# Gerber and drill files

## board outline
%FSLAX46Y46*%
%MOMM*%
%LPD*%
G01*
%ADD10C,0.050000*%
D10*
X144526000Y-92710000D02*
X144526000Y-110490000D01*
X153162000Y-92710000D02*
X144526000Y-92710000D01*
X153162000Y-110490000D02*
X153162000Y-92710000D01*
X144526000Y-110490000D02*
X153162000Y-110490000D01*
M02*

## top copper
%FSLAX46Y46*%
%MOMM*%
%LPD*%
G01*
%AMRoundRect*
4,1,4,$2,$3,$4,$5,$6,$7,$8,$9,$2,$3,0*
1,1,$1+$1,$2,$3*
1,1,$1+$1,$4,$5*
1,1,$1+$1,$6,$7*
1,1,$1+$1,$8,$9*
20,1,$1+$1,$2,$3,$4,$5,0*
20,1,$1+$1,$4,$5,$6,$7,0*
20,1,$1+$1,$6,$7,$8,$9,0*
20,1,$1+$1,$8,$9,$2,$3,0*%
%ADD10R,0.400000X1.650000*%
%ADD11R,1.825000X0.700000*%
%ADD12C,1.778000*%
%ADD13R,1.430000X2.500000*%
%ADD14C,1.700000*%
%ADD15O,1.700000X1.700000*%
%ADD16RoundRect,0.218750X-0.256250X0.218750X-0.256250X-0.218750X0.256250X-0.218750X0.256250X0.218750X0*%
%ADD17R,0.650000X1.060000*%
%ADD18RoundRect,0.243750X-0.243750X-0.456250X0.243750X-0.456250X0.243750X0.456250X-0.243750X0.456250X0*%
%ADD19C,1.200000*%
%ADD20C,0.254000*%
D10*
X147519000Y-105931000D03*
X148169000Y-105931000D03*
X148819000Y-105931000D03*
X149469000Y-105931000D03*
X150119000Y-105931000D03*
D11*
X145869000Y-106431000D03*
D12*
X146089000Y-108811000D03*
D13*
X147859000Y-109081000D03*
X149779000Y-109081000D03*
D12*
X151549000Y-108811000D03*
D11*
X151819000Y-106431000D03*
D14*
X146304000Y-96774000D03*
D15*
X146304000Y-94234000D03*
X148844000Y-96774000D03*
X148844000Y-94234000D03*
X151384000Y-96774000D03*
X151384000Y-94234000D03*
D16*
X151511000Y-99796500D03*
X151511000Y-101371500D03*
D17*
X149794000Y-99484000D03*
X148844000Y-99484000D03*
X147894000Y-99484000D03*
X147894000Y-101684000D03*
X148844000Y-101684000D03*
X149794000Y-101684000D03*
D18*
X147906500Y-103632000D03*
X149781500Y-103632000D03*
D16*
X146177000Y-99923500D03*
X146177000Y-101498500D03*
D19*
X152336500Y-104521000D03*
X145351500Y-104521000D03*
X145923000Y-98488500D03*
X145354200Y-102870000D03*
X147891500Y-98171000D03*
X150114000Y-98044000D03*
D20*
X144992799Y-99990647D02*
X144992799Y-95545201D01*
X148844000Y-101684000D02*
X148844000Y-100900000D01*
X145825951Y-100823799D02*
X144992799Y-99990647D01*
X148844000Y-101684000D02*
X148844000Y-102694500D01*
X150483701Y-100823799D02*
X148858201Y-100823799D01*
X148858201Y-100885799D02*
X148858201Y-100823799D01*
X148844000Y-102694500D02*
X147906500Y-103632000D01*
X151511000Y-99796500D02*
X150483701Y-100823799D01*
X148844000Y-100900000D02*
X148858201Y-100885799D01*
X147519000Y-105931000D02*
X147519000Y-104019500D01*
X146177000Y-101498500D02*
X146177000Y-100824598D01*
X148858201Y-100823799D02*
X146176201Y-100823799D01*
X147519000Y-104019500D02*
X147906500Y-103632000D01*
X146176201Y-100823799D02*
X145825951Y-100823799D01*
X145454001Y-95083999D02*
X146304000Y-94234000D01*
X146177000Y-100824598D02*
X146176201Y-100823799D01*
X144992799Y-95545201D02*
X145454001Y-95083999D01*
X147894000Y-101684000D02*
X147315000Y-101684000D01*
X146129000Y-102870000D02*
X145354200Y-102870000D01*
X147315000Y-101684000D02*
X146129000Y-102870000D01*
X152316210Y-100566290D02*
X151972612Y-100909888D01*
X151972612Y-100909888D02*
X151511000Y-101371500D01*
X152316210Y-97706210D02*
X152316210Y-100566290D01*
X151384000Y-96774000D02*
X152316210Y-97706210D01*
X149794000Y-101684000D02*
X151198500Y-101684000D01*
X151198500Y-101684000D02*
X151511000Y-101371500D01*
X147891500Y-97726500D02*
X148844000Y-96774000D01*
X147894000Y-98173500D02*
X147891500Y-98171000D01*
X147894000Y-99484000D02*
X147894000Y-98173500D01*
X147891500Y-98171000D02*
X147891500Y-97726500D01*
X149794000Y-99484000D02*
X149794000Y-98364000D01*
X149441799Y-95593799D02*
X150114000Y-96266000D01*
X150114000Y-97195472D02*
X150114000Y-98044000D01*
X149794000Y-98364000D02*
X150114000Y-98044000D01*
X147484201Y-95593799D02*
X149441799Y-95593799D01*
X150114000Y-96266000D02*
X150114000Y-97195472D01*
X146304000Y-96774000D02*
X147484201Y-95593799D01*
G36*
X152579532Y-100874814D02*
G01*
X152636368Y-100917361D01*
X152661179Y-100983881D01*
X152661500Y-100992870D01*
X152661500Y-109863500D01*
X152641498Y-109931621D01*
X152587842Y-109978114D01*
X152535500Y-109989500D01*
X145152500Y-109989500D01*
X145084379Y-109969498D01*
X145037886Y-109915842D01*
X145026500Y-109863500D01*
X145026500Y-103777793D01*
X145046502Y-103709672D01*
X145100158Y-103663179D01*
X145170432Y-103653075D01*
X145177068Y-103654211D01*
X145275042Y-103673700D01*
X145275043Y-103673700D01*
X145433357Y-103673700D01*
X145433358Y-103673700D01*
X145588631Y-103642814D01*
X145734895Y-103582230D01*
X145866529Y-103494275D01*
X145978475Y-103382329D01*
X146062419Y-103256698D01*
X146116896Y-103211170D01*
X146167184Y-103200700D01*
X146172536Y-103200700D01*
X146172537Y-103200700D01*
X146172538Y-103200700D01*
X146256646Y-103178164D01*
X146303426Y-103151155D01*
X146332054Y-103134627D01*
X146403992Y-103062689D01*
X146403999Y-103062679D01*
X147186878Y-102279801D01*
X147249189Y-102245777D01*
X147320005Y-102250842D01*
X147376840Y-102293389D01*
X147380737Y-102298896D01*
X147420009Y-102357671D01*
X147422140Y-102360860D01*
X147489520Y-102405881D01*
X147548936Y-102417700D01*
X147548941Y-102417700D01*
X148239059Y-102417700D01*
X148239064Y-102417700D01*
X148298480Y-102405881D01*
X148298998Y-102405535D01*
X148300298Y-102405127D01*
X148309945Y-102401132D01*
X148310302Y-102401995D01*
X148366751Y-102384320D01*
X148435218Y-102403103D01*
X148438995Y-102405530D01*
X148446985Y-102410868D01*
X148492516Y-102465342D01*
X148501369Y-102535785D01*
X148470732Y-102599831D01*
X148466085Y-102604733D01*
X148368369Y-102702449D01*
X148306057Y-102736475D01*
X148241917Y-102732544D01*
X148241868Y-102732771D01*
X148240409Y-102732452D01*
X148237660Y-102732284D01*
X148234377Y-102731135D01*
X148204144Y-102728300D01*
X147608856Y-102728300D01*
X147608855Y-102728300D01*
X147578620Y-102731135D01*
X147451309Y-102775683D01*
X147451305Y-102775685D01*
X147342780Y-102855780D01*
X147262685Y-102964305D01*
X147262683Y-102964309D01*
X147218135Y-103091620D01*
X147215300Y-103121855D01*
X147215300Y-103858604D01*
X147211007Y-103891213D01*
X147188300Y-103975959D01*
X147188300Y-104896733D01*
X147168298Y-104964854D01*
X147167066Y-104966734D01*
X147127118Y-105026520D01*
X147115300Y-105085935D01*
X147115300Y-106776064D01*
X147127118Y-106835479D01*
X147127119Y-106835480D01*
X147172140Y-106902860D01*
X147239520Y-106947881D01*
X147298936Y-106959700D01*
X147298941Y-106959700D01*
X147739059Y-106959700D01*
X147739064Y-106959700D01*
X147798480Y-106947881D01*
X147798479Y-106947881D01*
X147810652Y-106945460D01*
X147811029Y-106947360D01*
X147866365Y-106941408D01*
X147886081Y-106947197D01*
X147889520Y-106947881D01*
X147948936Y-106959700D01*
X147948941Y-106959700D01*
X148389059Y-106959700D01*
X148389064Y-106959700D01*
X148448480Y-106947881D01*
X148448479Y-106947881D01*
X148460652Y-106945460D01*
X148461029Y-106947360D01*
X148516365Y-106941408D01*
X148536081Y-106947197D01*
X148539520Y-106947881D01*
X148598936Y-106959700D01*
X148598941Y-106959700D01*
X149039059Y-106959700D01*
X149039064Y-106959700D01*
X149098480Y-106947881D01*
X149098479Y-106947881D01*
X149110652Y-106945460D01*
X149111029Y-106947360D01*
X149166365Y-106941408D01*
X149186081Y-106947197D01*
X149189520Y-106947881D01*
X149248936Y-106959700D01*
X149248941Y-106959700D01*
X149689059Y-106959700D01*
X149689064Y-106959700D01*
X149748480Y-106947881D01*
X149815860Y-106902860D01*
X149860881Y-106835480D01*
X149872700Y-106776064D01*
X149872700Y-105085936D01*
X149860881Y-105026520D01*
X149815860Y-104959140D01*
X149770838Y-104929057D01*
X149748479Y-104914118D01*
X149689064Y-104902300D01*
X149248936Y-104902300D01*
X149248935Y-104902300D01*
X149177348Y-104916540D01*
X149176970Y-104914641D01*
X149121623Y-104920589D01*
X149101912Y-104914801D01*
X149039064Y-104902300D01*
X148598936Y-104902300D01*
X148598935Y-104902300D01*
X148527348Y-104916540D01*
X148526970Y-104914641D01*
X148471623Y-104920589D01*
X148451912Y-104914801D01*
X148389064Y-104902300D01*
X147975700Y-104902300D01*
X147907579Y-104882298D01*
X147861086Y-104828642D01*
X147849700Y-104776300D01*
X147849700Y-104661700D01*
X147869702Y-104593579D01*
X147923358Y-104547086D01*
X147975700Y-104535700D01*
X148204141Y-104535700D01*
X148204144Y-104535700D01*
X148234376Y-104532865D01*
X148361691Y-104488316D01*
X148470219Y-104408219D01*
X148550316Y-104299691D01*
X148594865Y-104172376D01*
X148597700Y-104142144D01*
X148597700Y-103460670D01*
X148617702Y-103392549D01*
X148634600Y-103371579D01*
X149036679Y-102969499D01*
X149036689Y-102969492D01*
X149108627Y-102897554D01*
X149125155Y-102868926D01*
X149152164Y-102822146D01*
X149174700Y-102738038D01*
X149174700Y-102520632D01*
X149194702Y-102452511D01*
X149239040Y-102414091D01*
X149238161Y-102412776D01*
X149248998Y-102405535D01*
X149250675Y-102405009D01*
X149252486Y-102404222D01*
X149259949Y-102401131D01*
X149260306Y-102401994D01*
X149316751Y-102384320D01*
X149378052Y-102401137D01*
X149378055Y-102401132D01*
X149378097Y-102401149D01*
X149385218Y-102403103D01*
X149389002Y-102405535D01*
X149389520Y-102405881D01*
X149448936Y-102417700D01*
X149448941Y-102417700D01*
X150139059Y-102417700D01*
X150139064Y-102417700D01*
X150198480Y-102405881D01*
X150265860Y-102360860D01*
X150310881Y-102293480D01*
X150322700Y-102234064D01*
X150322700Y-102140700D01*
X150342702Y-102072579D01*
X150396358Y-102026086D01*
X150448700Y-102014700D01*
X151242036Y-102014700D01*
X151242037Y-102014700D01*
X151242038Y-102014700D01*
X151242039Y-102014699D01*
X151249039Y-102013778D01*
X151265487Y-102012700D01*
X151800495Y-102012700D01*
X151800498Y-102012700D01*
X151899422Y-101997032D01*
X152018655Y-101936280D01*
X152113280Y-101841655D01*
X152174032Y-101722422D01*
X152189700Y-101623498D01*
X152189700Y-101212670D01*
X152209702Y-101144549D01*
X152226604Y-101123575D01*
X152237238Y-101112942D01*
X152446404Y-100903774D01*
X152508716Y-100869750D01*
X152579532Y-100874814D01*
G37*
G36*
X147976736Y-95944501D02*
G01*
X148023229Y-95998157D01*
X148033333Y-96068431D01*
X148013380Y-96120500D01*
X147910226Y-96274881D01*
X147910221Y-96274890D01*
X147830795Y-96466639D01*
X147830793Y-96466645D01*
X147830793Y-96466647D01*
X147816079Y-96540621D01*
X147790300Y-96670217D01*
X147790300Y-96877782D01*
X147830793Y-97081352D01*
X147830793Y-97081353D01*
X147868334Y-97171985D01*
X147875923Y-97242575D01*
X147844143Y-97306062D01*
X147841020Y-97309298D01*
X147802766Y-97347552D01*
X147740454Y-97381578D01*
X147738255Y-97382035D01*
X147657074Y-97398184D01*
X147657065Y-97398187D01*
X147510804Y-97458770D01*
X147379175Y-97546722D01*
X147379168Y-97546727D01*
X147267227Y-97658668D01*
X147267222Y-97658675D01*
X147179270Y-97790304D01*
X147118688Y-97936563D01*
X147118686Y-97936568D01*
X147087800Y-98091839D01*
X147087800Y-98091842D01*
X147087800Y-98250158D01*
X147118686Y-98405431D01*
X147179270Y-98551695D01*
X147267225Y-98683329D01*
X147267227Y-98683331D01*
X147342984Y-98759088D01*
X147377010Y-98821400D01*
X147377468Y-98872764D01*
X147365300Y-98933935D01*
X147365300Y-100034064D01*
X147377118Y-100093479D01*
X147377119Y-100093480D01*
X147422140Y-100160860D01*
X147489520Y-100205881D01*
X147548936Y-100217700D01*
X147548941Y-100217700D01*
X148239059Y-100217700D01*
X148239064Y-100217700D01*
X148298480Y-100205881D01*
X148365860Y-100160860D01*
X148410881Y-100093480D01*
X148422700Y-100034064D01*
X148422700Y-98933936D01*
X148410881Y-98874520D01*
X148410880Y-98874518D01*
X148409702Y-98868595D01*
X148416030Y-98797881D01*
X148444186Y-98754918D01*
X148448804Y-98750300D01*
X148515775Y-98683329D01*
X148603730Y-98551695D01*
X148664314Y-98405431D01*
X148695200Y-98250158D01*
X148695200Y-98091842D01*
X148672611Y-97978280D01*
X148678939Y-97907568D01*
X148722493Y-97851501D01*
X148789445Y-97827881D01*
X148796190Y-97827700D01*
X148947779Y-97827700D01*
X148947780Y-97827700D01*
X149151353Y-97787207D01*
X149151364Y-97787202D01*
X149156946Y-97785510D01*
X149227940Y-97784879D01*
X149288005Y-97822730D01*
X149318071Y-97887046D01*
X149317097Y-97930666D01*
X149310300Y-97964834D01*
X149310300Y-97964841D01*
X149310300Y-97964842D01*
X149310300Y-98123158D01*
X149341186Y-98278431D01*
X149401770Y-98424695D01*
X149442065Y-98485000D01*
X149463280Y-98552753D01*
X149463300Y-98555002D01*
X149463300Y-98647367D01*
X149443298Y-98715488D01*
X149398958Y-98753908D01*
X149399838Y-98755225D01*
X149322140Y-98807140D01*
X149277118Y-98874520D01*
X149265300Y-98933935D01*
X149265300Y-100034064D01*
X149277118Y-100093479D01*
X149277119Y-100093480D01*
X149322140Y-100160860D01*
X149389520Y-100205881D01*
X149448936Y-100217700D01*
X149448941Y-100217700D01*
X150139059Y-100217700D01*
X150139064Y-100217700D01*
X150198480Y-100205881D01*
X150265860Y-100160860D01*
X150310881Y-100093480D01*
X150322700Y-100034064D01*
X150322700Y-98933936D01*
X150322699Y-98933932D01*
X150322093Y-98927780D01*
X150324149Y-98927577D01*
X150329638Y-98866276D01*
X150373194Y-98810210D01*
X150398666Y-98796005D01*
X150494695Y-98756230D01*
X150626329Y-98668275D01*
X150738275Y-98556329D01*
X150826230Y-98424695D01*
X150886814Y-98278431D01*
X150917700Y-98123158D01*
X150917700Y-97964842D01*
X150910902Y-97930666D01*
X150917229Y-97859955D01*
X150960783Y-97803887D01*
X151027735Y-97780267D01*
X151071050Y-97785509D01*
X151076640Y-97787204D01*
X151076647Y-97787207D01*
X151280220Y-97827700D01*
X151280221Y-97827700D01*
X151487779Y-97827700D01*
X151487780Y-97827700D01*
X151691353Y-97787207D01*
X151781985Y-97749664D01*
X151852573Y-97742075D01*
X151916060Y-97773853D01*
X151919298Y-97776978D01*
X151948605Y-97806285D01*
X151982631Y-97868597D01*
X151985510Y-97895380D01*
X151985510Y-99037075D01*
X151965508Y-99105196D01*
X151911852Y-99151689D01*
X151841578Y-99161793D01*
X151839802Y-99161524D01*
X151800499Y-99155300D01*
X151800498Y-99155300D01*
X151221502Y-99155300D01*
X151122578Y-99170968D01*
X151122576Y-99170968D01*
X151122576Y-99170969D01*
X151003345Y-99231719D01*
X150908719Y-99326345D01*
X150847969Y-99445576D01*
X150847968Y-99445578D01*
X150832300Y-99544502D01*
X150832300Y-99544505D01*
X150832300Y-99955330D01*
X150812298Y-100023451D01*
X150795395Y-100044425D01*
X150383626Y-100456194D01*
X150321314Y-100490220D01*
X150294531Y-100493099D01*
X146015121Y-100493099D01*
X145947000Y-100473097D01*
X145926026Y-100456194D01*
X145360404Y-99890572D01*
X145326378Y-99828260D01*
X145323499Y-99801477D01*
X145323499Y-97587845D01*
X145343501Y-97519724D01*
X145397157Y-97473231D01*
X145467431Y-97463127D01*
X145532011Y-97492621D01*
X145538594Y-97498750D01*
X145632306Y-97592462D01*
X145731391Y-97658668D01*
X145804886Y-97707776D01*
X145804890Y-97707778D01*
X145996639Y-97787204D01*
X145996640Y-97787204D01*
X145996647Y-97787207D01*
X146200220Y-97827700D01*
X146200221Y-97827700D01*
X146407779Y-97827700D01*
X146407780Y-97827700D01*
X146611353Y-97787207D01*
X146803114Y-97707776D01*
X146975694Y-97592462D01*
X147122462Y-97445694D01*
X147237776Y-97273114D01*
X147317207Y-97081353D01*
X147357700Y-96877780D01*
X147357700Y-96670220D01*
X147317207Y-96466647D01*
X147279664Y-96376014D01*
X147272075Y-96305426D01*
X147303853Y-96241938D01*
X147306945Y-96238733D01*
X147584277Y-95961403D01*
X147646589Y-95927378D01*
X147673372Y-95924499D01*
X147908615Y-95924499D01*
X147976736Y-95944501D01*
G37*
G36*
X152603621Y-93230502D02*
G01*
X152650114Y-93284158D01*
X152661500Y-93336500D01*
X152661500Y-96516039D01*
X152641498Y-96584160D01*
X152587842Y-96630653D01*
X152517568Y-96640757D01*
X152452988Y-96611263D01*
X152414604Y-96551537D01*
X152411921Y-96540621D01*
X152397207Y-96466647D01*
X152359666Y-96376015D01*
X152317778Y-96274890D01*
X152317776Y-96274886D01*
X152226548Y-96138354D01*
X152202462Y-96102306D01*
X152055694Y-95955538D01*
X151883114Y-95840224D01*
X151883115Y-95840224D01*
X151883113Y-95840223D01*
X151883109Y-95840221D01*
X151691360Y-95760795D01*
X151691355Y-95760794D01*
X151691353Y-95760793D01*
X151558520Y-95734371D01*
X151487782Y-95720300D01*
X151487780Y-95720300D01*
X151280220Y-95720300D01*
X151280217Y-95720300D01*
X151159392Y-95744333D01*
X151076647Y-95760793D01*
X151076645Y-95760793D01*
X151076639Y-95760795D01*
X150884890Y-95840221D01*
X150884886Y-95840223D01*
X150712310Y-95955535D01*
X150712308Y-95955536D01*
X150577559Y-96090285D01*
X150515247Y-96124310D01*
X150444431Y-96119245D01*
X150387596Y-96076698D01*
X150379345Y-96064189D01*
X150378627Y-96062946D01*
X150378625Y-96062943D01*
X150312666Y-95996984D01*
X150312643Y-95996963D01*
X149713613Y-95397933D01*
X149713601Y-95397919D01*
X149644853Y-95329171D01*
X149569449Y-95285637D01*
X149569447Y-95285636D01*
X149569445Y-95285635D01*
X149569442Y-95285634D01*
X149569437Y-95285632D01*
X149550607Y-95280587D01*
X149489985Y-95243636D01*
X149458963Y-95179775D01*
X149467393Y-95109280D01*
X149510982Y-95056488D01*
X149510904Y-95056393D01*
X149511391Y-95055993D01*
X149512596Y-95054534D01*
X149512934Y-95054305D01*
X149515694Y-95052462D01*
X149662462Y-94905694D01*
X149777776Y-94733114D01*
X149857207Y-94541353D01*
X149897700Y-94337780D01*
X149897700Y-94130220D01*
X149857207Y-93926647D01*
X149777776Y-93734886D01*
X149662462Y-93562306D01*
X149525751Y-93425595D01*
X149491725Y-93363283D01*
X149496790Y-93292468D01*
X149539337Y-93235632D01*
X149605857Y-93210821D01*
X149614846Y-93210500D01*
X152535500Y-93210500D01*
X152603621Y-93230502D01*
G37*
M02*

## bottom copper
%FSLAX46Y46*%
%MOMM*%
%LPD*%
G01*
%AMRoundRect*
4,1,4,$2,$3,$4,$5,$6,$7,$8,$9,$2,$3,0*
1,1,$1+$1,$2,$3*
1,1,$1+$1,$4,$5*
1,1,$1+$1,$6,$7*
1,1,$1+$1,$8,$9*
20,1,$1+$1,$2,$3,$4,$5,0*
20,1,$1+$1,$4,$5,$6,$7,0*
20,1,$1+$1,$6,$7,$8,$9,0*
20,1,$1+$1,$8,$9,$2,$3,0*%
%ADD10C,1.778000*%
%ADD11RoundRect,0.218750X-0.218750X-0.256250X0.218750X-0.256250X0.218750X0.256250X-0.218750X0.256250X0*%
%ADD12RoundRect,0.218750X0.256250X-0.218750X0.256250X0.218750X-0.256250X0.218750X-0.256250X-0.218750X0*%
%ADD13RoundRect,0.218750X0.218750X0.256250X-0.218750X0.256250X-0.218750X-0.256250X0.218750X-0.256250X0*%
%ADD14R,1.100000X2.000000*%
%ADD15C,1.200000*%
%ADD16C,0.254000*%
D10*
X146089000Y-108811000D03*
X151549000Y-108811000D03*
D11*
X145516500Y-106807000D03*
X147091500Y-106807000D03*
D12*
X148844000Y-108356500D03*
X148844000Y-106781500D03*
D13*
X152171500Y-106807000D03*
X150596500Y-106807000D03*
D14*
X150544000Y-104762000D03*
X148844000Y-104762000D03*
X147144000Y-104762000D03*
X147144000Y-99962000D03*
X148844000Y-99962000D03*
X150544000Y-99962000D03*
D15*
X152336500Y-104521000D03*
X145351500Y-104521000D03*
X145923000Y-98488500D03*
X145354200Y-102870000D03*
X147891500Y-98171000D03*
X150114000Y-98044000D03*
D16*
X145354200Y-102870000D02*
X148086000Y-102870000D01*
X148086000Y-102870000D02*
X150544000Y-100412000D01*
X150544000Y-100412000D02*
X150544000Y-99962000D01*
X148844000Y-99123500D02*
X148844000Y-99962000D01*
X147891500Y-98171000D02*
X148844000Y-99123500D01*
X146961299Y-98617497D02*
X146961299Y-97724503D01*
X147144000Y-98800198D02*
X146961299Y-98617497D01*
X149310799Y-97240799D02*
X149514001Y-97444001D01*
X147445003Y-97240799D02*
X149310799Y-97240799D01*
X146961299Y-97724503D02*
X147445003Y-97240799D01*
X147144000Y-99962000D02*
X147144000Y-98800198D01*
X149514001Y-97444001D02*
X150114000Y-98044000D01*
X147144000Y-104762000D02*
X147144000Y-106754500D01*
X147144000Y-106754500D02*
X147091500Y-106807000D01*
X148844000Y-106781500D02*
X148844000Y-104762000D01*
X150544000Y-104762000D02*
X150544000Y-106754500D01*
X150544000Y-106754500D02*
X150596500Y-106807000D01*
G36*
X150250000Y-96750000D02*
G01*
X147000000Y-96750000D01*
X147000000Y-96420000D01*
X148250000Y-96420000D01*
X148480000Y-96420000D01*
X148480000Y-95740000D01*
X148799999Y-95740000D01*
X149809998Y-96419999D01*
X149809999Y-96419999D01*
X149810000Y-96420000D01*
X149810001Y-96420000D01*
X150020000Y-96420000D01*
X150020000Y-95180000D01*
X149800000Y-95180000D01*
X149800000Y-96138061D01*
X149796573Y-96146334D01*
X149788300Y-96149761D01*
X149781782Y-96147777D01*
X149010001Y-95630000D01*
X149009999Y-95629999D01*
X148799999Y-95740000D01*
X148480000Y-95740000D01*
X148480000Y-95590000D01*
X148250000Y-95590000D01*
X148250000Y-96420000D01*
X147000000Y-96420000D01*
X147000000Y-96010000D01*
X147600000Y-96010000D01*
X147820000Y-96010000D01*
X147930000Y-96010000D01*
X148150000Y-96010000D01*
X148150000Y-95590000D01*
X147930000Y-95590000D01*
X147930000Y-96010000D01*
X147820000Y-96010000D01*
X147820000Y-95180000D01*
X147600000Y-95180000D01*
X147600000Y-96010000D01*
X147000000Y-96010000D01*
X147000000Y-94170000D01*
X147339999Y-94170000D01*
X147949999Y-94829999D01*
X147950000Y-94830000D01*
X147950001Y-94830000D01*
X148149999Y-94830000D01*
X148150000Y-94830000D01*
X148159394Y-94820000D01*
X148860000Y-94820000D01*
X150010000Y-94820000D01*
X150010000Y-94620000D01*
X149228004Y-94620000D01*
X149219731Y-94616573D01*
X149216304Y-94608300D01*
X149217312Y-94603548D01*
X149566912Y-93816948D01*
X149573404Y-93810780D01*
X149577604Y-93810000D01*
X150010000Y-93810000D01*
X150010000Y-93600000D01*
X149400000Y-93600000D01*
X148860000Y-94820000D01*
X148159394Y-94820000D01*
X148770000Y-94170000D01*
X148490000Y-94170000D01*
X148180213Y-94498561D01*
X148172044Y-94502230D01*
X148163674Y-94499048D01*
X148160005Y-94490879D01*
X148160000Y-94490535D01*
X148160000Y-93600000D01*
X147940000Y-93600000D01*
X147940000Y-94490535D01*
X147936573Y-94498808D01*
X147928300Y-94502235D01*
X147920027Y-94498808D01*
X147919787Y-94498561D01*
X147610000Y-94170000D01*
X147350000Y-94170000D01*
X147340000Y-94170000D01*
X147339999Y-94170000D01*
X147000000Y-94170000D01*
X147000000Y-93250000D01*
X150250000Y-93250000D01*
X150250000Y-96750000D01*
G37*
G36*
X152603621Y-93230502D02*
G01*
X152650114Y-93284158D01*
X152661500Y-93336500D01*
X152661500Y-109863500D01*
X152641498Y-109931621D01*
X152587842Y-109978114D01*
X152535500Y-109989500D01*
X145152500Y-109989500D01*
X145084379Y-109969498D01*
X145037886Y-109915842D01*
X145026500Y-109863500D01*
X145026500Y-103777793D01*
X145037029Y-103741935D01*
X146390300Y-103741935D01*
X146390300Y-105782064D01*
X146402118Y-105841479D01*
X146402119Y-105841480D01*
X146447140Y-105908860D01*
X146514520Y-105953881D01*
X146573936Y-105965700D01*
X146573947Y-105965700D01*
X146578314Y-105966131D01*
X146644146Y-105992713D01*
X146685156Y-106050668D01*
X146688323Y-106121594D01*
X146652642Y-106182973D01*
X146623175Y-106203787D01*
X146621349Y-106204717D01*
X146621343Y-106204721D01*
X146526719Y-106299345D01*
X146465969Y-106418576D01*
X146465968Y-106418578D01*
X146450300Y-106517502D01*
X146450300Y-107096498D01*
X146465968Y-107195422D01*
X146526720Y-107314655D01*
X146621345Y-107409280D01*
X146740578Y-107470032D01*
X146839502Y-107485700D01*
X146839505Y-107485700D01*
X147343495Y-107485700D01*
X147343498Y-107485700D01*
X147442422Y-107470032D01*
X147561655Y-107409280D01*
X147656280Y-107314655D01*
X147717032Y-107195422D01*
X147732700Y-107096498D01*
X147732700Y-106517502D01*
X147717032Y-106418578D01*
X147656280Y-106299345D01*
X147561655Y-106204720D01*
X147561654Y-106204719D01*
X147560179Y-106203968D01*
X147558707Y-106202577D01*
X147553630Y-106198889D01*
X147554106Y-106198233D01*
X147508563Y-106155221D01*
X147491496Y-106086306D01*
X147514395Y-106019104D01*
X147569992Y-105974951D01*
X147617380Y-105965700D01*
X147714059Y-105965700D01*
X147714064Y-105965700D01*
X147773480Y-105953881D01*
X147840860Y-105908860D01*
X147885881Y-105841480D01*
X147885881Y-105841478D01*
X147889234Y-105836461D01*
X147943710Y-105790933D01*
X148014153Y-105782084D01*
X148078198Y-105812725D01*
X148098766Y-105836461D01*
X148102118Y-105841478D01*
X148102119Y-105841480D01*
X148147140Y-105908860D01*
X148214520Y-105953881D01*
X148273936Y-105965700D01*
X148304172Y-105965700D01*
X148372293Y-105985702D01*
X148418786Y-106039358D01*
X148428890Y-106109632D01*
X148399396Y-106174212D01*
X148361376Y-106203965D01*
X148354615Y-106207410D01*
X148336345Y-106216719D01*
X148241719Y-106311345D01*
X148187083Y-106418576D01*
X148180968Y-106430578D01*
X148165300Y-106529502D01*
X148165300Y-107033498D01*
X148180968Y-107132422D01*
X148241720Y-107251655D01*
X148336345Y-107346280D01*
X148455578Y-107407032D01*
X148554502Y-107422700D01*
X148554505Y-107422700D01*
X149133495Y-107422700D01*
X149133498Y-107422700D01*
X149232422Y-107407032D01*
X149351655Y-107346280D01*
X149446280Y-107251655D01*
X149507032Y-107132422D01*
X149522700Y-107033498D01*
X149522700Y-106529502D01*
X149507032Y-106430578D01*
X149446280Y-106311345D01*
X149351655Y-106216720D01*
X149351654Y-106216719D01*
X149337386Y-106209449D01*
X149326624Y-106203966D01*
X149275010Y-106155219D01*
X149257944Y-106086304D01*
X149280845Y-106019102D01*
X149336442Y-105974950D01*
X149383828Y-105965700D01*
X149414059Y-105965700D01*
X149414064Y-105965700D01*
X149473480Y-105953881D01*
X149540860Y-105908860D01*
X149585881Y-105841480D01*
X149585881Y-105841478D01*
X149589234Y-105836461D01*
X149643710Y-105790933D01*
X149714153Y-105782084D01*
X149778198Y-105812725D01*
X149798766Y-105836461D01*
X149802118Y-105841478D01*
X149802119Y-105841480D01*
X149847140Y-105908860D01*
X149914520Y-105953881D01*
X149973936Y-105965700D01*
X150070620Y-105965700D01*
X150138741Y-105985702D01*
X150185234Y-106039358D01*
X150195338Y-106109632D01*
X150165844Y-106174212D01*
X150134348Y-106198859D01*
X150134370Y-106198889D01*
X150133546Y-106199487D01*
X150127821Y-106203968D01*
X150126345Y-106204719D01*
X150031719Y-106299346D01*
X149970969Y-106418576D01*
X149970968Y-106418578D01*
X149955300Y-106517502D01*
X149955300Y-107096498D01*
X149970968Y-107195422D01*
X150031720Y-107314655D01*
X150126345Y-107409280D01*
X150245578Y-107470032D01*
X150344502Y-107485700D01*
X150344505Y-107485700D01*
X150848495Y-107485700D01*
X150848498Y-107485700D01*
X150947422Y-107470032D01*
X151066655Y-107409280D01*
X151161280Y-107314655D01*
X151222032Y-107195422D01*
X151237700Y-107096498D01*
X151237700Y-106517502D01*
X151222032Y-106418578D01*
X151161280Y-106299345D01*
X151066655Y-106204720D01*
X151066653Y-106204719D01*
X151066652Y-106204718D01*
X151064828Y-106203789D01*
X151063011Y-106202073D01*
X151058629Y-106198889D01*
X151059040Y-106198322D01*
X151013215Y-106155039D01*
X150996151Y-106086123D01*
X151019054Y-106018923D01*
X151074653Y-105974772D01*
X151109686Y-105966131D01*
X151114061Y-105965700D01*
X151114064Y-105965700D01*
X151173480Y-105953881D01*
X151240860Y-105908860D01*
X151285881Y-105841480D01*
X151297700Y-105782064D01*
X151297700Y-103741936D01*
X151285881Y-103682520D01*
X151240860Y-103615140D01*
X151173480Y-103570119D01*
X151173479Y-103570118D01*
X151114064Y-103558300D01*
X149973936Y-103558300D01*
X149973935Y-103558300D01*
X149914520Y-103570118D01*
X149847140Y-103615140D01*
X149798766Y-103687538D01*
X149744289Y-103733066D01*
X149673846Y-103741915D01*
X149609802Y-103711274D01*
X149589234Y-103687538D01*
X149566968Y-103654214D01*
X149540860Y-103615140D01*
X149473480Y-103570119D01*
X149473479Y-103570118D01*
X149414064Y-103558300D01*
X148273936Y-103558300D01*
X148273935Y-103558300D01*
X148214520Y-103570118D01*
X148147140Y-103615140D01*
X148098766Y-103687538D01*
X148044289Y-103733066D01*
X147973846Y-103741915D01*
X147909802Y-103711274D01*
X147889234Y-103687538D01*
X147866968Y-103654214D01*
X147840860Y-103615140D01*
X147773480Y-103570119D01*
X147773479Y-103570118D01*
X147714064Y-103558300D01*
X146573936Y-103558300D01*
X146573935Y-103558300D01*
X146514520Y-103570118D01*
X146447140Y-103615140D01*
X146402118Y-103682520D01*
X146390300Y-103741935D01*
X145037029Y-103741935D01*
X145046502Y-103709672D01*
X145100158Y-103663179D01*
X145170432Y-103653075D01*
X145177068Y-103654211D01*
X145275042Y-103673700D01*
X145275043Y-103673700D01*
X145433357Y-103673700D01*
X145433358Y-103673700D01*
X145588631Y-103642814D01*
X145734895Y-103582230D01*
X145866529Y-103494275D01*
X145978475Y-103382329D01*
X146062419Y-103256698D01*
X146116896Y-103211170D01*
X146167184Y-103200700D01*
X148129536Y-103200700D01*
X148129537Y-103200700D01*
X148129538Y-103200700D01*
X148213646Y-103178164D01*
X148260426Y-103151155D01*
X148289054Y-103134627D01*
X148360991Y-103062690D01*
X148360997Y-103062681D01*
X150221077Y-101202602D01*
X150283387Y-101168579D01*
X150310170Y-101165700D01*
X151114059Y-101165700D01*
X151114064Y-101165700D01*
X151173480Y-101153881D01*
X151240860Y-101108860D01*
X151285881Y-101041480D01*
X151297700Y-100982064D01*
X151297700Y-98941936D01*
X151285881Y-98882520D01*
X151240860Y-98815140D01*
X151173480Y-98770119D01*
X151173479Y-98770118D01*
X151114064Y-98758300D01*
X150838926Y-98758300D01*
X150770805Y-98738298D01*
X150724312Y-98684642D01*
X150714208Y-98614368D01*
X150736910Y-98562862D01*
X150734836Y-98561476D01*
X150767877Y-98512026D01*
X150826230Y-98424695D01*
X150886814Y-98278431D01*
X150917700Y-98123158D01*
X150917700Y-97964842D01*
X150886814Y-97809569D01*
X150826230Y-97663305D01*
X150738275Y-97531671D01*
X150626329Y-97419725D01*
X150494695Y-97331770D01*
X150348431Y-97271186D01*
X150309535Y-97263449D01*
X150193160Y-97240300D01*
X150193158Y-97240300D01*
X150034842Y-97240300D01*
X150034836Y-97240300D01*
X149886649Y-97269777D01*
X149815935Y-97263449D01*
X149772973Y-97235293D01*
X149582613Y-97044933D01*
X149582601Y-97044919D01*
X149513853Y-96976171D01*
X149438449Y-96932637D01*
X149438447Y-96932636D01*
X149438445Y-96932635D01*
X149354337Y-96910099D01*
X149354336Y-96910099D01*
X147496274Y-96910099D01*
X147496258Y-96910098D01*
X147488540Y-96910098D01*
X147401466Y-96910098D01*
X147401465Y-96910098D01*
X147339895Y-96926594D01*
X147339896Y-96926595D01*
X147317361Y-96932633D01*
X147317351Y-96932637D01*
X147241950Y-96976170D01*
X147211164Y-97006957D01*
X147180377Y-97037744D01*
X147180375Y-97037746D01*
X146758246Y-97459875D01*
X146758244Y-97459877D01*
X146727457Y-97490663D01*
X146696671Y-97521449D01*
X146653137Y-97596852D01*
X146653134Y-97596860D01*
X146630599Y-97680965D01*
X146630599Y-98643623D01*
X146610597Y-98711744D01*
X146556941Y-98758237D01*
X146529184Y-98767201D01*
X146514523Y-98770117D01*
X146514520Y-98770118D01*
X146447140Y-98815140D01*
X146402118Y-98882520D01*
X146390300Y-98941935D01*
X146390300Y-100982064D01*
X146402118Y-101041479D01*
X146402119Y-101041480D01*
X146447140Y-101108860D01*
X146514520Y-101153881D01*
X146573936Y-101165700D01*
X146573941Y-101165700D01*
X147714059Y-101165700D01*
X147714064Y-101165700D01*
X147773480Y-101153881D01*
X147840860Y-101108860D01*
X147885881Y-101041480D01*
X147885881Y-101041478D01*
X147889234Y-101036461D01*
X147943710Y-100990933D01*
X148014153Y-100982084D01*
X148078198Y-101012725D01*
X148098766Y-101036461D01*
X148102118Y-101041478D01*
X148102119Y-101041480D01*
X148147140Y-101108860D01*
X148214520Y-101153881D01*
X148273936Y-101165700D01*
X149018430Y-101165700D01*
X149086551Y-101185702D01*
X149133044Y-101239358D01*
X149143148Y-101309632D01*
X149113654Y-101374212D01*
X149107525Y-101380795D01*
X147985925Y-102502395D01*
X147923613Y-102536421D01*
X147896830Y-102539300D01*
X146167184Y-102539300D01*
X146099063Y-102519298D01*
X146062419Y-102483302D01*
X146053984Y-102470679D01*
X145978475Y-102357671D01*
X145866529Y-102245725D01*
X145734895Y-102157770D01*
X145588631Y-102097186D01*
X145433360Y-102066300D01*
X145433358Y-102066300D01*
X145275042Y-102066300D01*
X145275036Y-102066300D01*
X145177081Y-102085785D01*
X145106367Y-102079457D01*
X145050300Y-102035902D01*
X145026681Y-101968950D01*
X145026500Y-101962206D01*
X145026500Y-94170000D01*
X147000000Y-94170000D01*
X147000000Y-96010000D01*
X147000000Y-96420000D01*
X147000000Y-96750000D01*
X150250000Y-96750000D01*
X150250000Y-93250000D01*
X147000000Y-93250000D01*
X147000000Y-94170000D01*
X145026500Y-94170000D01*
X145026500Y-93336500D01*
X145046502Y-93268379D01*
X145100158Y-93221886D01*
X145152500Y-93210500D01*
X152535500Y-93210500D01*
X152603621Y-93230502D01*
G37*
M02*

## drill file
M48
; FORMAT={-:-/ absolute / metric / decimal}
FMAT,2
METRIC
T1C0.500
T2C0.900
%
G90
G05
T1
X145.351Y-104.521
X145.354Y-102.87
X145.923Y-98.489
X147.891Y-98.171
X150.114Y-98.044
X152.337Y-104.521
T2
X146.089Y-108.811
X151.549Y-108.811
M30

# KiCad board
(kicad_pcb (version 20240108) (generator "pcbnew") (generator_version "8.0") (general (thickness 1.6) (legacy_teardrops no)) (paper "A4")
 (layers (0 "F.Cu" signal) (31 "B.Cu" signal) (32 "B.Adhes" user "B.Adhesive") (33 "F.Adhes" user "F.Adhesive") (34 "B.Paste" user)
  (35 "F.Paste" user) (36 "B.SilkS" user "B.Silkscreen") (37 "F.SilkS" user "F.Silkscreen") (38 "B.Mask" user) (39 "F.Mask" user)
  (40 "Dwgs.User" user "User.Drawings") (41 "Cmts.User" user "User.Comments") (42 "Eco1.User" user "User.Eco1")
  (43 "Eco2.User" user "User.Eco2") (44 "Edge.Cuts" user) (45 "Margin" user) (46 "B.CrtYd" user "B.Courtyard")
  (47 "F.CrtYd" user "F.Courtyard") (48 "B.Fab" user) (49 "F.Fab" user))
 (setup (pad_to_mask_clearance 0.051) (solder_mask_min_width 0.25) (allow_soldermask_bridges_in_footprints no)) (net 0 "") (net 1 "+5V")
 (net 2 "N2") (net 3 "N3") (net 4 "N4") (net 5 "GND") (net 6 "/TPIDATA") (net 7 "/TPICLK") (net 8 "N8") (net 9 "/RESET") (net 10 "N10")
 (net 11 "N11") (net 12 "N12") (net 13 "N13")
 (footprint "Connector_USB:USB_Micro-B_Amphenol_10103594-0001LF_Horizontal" (layer "F.Cu") (at 148.844 107.696)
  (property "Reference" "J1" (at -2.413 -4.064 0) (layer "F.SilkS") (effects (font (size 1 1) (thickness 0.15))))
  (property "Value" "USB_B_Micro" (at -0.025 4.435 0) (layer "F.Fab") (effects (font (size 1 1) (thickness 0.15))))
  (pad "1" smd rect (at -1.325 -1.765 90) (size 1.65 0.4) (layers "F.Cu" "F.Paste" "F.Mask") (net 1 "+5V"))
  (pad "2" smd rect (at -0.675 -1.765 90) (size 1.65 0.4) (layers "F.Cu" "F.Paste" "F.Mask") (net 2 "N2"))
  (pad "3" smd rect (at -0.025 -1.765 90) (size 1.65 0.4) (layers "F.Cu" "F.Paste" "F.Mask") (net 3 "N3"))
  (pad "4" smd rect (at 0.625 -1.765 90) (size 1.65 0.4) (layers "F.Cu" "F.Paste" "F.Mask") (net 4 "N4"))
  (pad "5" smd rect (at 1.275 -1.765 90) (size 1.65 0.4) (layers "F.Cu" "F.Paste" "F.Mask") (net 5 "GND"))
  (pad "6" smd rect (at -2.975 -1.265) (size 1.825 0.7) (layers "F.Cu" "F.Paste" "F.Mask") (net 5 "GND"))
  (pad "6" thru_hole circle (at -2.755 1.115 90) (size 1.778 1.778) (drill 0.9) (layers "*.Cu" "*.Mask") (remove_unused_layers no)
   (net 5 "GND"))
  (pad "6" smd rect (at -0.985 1.385 90) (size 2.5 1.43) (layers "F.Cu" "F.Paste" "F.Mask") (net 5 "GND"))
  (pad "6" smd rect (at 0.935 1.385 90) (size 2.5 1.43) (layers "F.Cu" "F.Paste" "F.Mask") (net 5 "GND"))
  (pad "6" thru_hole circle (at 2.705 1.115 90) (size 1.778 1.778) (drill 0.9) (layers "*.Cu" "*.Mask") (remove_unused_layers no)
   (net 5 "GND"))
  (pad "6" smd rect (at 2.975 -1.265) (size 1.825 0.7) (layers "F.Cu" "F.Paste" "F.Mask") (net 5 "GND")))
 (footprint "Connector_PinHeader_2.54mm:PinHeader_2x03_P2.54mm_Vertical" (layer "F.Cu") (at 146.304 96.774 90)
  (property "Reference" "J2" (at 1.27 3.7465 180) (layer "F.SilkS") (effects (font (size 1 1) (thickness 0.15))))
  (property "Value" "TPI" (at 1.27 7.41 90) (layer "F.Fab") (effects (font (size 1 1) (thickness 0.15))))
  (pad "1" smd circle (at 0 0 90) (size 1.7 1.7) (layers "F.Cu" "F.Paste" "F.Mask") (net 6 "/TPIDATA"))
  (pad "2" smd oval (at 2.54 0 90) (size 1.7 1.7) (layers "F.Cu" "F.Paste" "F.Mask") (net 1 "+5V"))
  (pad "3" smd oval (at 0 2.54 90) (size 1.7 1.7) (layers "F.Cu" "F.Paste" "F.Mask") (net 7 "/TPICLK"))
  (pad "4" smd oval (at 2.54 2.54 90) (size 1.7 1.7) (layers "F.Cu" "F.Paste" "F.Mask") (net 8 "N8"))
  (pad "5" smd oval (at 0 5.08 90) (size 1.7 1.7) (layers "F.Cu" "F.Paste" "F.Mask") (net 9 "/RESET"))
  (pad "6" smd oval (at 2.54 5.08 90) (size 1.7 1.7) (layers "F.Cu" "F.Paste" "F.Mask") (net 5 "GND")))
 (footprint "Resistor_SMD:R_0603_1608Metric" (layer "F.Cu") (at 151.511 100.584 -90)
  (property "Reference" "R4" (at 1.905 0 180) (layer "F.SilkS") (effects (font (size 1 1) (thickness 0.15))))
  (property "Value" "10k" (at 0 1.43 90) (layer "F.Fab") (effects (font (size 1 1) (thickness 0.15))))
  (pad "1" smd roundrect (at -0.7875 0 270) (size 0.875 0.95) (layers "F.Cu" "F.Paste" "F.Mask") (roundrect_rratio 0.25) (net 1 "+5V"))
  (pad "2" smd roundrect (at 0.7875 0 270) (size 0.875 0.95) (layers "F.Cu" "F.Paste" "F.Mask") (roundrect_rratio 0.25) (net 9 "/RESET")))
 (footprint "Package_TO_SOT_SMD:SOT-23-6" (layer "F.Cu") (at 148.844 100.584 -90)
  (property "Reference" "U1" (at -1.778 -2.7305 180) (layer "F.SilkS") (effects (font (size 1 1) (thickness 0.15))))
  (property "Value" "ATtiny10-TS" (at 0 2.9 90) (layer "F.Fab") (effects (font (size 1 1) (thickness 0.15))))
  (pad "1" smd rect (at -1.1 -0.95 270) (size 1.06 0.65) (layers "F.Cu" "F.Paste" "F.Mask") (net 6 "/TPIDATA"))
  (pad "2" smd rect (at -1.1 0 270) (size 1.06 0.65) (layers "F.Cu" "F.Paste" "F.Mask") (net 5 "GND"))
  (pad "3" smd rect (at -1.1 0.95 270) (size 1.06 0.65) (layers "F.Cu" "F.Paste" "F.Mask") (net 7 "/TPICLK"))
  (pad "4" smd rect (at 1.1 0.95 270) (size 1.06 0.65) (layers "F.Cu" "F.Paste" "F.Mask") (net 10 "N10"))
  (pad "5" smd rect (at 1.1 0 270) (size 1.06 0.65) (layers "F.Cu" "F.Paste" "F.Mask") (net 1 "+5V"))
  (pad "6" smd rect (at 1.1 -0.95 270) (size 1.06 0.65) (layers "F.Cu" "F.Paste" "F.Mask") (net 9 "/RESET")))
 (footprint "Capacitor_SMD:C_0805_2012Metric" (layer "F.Cu") (at 148.844 103.632)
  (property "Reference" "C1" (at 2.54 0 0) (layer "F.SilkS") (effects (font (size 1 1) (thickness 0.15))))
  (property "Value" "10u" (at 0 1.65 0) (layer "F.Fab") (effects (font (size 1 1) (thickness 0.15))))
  (pad "1" smd roundrect (at -0.9375 0) (size 0.975 1.4) (layers "F.Cu" "F.Paste" "F.Mask") (roundrect_rratio 0.25) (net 1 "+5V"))
  (pad "2" smd roundrect (at 0.9375 0) (size 0.975 1.4) (layers "F.Cu" "F.Paste" "F.Mask") (roundrect_rratio 0.25) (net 5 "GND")))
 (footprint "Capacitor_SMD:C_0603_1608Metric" (layer "F.Cu") (at 146.177 100.711 -90)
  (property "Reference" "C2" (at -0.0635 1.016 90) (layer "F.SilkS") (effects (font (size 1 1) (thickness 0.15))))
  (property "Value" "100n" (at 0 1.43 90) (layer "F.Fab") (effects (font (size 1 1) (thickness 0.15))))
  (pad "1" smd roundrect (at -0.7875 0 270) (size 0.875 0.95) (layers "F.Cu" "F.Paste" "F.Mask") (roundrect_rratio 0.25) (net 5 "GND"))
  (pad "2" smd roundrect (at 0.7875 0 270) (size 0.875 0.95) (layers "F.Cu" "F.Paste" "F.Mask") (roundrect_rratio 0.25) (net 1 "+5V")))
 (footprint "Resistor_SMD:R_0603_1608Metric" (layer "B.Cu") (at 146.304 106.807)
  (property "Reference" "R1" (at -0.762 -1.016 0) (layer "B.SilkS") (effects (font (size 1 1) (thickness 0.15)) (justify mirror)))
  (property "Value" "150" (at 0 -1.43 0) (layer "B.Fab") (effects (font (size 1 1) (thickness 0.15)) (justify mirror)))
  (pad "1" smd roundrect (at -0.7875 0) (size 0.875 0.95) (layers "B.Cu" "B.Paste" "B.Mask") (roundrect_rratio 0.25) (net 5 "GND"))
  (pad "2" smd roundrect (at 0.7875 0) (size 0.875 0.95) (layers "B.Cu" "B.Paste" "B.Mask") (roundrect_rratio 0.25) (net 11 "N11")))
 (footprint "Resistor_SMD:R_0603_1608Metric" (layer "B.Cu") (at 148.844 107.569 90)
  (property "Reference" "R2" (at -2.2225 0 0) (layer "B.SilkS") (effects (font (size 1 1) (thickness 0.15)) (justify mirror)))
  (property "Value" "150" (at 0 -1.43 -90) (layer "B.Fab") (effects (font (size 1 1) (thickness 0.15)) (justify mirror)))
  (pad "1" smd roundrect (at -0.7875 0 90) (size 0.875 0.95) (layers "B.Cu" "B.Paste" "B.Mask") (roundrect_rratio 0.25) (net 5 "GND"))
  (pad "2" smd roundrect (at 0.7875 0 90) (size 0.875 0.95) (layers "B.Cu" "B.Paste" "B.Mask") (roundrect_rratio 0.25) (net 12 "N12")))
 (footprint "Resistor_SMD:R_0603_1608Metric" (layer "B.Cu") (at 151.384 106.807 180)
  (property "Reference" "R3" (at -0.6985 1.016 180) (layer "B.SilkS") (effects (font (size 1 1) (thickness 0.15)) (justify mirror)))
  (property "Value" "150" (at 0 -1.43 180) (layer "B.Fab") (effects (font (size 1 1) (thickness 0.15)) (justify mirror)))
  (pad "1" smd roundrect (at -0.7875 0 180) (size 0.875 0.95) (layers "B.Cu" "B.Paste" "B.Mask") (roundrect_rratio 0.25) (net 5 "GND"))
  (pad "2" smd roundrect (at 0.7875 0 180) (size 0.875 0.95) (layers "B.Cu" "B.Paste" "B.Mask") (roundrect_rratio 0.25) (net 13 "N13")))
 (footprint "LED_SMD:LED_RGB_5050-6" (layer "B.Cu") (at 148.844 102.362 90)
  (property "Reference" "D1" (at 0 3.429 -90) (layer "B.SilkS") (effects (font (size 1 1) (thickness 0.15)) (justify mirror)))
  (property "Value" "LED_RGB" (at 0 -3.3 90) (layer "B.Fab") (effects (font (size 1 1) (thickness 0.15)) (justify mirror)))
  (pad "1" smd rect (at -2.4 1.7) (size 1.1 2) (layers "B.Cu" "B.Paste" "B.Mask") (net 13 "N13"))
  (pad "2" smd rect (at -2.4 0) (size 1.1 2) (layers "B.Cu" "B.Paste" "B.Mask") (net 12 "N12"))
  (pad "3" smd rect (at -2.4 -1.7) (size 1.1 2) (layers "B.Cu" "B.Paste" "B.Mask") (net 11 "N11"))
  (pad "4" smd rect (at 2.4 -1.7) (size 1.1 2) (layers "B.Cu" "B.Paste" "B.Mask") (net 6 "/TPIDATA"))
  (pad "5" smd rect (at 2.4 0) (size 1.1 2) (layers "B.Cu" "B.Paste" "B.Mask") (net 7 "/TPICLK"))
  (pad "6" smd rect (at 2.4 1.7) (size 1.1 2) (layers "B.Cu" "B.Paste" "B.Mask") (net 10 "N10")))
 (gr_line (start 144.526 92.71) (end 144.526 110.49) (stroke (width 0.05) (type solid)) (layer "Edge.Cuts"))
 (gr_line (start 153.162 92.71) (end 144.526 92.71) (stroke (width 0.05) (type solid)) (layer "Edge.Cuts"))
 (gr_line (start 153.162 110.49) (end 153.162 92.71) (stroke (width 0.05) (type solid)) (layer "Edge.Cuts"))
 (gr_line (start 144.526 110.49) (end 153.162 110.49) (stroke (width 0.05) (type solid)) (layer "Edge.Cuts"))
 (via (at 152.3365 104.521) (size 1.2) (drill 0.5) (layers "F.Cu" "B.Cu") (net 5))
 (via (at 145.3515 104.521) (size 1.2) (drill 0.5) (layers "F.Cu" "B.Cu") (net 5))
 (via (at 145.923 98.4885) (size 1.2) (drill 0.5) (layers "F.Cu" "B.Cu") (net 5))
 (segment (start 144.992799 99.990647) (end 144.992799 95.545201) (width 0.254) (layer "F.Cu") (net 1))
 (segment (start 148.844 101.684) (end 148.844 100.9) (width 0.254) (layer "F.Cu") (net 1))
 (segment (start 145.825951 100.823799) (end 144.992799 99.990647) (width 0.254) (layer "F.Cu") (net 1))
 (segment (start 148.844 101.684) (end 148.844 102.6945) (width 0.254) (layer "F.Cu") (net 1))
 (segment (start 150.483701 100.823799) (end 148.858201 100.823799) (width 0.254) (layer "F.Cu") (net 1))
 (segment (start 148.858201 100.885799) (end 148.858201 100.823799) (width 0.254) (layer "F.Cu") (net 1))
 (segment (start 148.844 102.6945) (end 147.9065 103.632) (width 0.254) (layer "F.Cu") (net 1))
 (segment (start 151.511 99.7965) (end 150.483701 100.823799) (width 0.254) (layer "F.Cu") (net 1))
 (segment (start 148.844 100.9) (end 148.858201 100.885799) (width 0.254) (layer "F.Cu") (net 1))
 (segment (start 147.519 105.931) (end 147.519 104.0195) (width 0.254) (layer "F.Cu") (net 1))
 (segment (start 146.177 101.4985) (end 146.177 100.824598) (width 0.254) (layer "F.Cu") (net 1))
 (segment (start 148.858201 100.823799) (end 146.176201 100.823799) (width 0.254) (layer "F.Cu") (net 1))
 (segment (start 147.519 104.0195) (end 147.9065 103.632) (width 0.254) (layer "F.Cu") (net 1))
 (segment (start 146.176201 100.823799) (end 145.825951 100.823799) (width 0.254) (layer "F.Cu") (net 1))
 (segment (start 145.454001 95.083999) (end 146.304 94.234) (width 0.254) (layer "F.Cu") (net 1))
 (segment (start 146.177 100.824598) (end 146.176201 100.823799) (width 0.254) (layer "F.Cu") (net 1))
 (segment (start 144.992799 95.545201) (end 145.454001 95.083999) (width 0.254) (layer "F.Cu") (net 1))
 (segment (start 147.894 101.684) (end 147.315 101.684) (width 0.254) (layer "F.Cu") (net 10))
 (segment (start 146.129 102.87) (end 145.3542 102.87) (width 0.254) (layer "F.Cu") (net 10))
 (segment (start 147.315 101.684) (end 146.129 102.87) (width 0.254) (layer "F.Cu") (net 10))
 (via (at 145.3542 102.87) (size 1.2) (drill 0.5) (layers "F.Cu" "B.Cu") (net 10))
 (segment (start 145.3542 102.87) (end 148.086 102.87) (width 0.254) (layer "B.Cu") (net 10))
 (segment (start 148.086 102.87) (end 150.544 100.412) (width 0.254) (layer "B.Cu") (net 10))
 (segment (start 150.544 100.412) (end 150.544 99.962) (width 0.254) (layer "B.Cu") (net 10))
 (segment (start 152.31621 100.56629) (end 151.972612 100.909888) (width 0.254) (layer "F.Cu") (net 9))
 (segment (start 151.972612 100.909888) (end 151.511 101.3715) (width 0.254) (layer "F.Cu") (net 9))
 (segment (start 152.31621 97.70621) (end 152.31621 100.56629) (width 0.254) (layer "F.Cu") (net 9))
 (segment (start 151.384 96.774) (end 152.31621 97.70621) (width 0.254) (layer "F.Cu") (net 9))
 (segment (start 149.794 101.684) (end 151.1985 101.684) (width 0.254) (layer "F.Cu") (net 9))
 (segment (start 151.1985 101.684) (end 151.511 101.3715) (width 0.254) (layer "F.Cu") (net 9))
 (segment (start 147.8915 97.7265) (end 148.844 96.774) (width 0.254) (layer "F.Cu") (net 7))
 (segment (start 147.894 98.1735) (end 147.8915 98.171) (width 0.254) (layer "F.Cu") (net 7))
 (segment (start 147.894 99.484) (end 147.894 98.1735) (width 0.254) (layer "F.Cu") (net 7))
 (segment (start 147.8915 98.171) (end 147.8915 97.7265) (width 0.254) (layer "F.Cu") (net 7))
 (via (at 147.8915 98.171) (size 1.2) (drill 0.5) (layers "F.Cu" "B.Cu") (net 7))
 (segment (start 148.844 99.1235) (end 148.844 99.962) (width 0.254) (layer "B.Cu") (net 7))
 (segment (start 147.8915 98.171) (end 148.844 99.1235) (width 0.254) (layer "B.Cu") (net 7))
 (segment (start 149.794 99.484) (end 149.794 98.364) (width 0.254) (layer "F.Cu") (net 6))
 (segment (start 149.441799 95.593799) (end 150.114 96.266) (width 0.254) (layer "F.Cu") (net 6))
 (segment (start 150.114 97.195472) (end 150.114 98.044) (width 0.254) (layer "F.Cu") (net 6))
 (segment (start 149.794 98.364) (end 150.114 98.044) (width 0.254) (layer "F.Cu") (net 6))
 (segment (start 147.484201 95.593799) (end 149.441799 95.593799) (width 0.254) (layer "F.Cu") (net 6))
 (segment (start 150.114 96.266) (end 150.114 97.195472) (width 0.254) (layer "F.Cu") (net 6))
 (segment (start 146.304 96.774) (end 147.484201 95.593799) (width 0.254) (layer "F.Cu") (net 6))
 (via (at 150.114 98.044) (size 1.2) (drill 0.5) (layers "F.Cu" "B.Cu") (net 6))
 (segment (start 146.961299 98.617497) (end 146.961299 97.724503) (width 0.254) (layer "B.Cu") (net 6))
 (segment (start 147.144 98.800198) (end 146.961299 98.617497) (width 0.254) (layer "B.Cu") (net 6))
 (segment (start 149.310799 97.240799) (end 149.514001 97.444001) (width 0.254) (layer "B.Cu") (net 6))
 (segment (start 147.445003 97.240799) (end 149.310799 97.240799) (width 0.254) (layer "B.Cu") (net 6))
 (segment (start 146.961299 97.724503) (end 147.445003 97.240799) (width 0.254) (layer "B.Cu") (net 6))
 (segment (start 147.144 99.962) (end 147.144 98.800198) (width 0.254) (layer "B.Cu") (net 6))
 (segment (start 149.514001 97.444001) (end 150.114 98.044) (width 0.254) (layer "B.Cu") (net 6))
 (segment (start 147.144 104.762) (end 147.144 106.7545) (width 0.254) (layer "B.Cu") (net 11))
 (segment (start 147.144 106.7545) (end 147.0915 106.807) (width 0.254) (layer "B.Cu") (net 11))
 (segment (start 148.844 106.7815) (end 148.844 104.762) (width 0.254) (layer "B.Cu") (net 12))
 (segment (start 150.544 104.762) (end 150.544 106.7545) (width 0.254) (layer "B.Cu") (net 13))
 (segment (start 150.544 106.7545) (end 150.5965 106.807) (width 0.254) (layer "B.Cu") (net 13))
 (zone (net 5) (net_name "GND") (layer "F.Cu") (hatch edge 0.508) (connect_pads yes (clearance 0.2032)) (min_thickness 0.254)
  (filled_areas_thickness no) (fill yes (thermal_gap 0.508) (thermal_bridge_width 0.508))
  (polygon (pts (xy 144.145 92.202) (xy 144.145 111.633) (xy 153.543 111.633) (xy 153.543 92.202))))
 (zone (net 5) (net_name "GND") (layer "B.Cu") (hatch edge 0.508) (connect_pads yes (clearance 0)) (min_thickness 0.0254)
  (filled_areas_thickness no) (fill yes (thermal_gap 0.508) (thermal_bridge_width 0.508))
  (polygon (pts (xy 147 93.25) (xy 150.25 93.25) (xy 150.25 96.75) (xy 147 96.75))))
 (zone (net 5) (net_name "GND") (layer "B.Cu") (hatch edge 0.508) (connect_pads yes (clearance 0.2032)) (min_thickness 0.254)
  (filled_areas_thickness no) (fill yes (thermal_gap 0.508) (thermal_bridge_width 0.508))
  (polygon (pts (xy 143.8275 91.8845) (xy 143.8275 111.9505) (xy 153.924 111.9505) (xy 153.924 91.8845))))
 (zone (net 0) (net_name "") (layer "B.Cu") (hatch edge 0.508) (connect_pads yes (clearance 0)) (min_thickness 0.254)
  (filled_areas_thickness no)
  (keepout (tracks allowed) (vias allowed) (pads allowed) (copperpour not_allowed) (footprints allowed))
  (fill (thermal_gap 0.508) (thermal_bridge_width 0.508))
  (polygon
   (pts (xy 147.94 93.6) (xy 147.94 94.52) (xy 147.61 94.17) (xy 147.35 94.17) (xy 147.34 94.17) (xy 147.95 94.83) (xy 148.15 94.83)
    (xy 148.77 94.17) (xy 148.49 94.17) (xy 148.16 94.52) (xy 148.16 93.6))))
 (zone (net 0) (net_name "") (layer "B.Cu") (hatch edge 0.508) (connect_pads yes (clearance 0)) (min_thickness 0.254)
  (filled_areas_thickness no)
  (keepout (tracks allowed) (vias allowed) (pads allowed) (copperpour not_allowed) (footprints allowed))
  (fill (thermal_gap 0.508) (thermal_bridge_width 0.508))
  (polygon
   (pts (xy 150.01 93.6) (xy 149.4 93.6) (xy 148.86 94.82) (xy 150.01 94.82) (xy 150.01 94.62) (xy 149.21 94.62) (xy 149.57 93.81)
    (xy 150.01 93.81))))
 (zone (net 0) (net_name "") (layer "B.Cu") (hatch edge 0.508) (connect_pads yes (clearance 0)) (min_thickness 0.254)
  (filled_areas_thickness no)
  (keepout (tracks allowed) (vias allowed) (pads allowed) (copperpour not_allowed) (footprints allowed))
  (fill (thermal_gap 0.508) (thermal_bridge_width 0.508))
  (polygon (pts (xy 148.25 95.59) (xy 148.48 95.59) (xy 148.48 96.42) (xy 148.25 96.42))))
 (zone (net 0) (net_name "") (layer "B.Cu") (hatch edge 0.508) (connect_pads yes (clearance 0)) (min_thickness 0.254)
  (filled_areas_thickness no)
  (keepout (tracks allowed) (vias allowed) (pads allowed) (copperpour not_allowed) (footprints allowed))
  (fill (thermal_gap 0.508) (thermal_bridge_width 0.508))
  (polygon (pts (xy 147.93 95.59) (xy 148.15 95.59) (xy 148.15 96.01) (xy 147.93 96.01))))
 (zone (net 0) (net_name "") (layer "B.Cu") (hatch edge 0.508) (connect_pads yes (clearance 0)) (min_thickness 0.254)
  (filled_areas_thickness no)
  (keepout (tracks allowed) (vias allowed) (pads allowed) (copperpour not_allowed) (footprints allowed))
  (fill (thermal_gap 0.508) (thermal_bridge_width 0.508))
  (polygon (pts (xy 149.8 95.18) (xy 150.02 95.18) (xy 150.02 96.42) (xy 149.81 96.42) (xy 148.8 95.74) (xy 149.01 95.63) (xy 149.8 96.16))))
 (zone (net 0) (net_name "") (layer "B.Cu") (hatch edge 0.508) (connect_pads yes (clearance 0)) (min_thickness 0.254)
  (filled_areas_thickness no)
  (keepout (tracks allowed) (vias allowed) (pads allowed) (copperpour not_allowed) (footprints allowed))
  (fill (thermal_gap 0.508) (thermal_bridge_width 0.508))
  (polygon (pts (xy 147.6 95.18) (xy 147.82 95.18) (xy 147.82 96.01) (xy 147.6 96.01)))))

